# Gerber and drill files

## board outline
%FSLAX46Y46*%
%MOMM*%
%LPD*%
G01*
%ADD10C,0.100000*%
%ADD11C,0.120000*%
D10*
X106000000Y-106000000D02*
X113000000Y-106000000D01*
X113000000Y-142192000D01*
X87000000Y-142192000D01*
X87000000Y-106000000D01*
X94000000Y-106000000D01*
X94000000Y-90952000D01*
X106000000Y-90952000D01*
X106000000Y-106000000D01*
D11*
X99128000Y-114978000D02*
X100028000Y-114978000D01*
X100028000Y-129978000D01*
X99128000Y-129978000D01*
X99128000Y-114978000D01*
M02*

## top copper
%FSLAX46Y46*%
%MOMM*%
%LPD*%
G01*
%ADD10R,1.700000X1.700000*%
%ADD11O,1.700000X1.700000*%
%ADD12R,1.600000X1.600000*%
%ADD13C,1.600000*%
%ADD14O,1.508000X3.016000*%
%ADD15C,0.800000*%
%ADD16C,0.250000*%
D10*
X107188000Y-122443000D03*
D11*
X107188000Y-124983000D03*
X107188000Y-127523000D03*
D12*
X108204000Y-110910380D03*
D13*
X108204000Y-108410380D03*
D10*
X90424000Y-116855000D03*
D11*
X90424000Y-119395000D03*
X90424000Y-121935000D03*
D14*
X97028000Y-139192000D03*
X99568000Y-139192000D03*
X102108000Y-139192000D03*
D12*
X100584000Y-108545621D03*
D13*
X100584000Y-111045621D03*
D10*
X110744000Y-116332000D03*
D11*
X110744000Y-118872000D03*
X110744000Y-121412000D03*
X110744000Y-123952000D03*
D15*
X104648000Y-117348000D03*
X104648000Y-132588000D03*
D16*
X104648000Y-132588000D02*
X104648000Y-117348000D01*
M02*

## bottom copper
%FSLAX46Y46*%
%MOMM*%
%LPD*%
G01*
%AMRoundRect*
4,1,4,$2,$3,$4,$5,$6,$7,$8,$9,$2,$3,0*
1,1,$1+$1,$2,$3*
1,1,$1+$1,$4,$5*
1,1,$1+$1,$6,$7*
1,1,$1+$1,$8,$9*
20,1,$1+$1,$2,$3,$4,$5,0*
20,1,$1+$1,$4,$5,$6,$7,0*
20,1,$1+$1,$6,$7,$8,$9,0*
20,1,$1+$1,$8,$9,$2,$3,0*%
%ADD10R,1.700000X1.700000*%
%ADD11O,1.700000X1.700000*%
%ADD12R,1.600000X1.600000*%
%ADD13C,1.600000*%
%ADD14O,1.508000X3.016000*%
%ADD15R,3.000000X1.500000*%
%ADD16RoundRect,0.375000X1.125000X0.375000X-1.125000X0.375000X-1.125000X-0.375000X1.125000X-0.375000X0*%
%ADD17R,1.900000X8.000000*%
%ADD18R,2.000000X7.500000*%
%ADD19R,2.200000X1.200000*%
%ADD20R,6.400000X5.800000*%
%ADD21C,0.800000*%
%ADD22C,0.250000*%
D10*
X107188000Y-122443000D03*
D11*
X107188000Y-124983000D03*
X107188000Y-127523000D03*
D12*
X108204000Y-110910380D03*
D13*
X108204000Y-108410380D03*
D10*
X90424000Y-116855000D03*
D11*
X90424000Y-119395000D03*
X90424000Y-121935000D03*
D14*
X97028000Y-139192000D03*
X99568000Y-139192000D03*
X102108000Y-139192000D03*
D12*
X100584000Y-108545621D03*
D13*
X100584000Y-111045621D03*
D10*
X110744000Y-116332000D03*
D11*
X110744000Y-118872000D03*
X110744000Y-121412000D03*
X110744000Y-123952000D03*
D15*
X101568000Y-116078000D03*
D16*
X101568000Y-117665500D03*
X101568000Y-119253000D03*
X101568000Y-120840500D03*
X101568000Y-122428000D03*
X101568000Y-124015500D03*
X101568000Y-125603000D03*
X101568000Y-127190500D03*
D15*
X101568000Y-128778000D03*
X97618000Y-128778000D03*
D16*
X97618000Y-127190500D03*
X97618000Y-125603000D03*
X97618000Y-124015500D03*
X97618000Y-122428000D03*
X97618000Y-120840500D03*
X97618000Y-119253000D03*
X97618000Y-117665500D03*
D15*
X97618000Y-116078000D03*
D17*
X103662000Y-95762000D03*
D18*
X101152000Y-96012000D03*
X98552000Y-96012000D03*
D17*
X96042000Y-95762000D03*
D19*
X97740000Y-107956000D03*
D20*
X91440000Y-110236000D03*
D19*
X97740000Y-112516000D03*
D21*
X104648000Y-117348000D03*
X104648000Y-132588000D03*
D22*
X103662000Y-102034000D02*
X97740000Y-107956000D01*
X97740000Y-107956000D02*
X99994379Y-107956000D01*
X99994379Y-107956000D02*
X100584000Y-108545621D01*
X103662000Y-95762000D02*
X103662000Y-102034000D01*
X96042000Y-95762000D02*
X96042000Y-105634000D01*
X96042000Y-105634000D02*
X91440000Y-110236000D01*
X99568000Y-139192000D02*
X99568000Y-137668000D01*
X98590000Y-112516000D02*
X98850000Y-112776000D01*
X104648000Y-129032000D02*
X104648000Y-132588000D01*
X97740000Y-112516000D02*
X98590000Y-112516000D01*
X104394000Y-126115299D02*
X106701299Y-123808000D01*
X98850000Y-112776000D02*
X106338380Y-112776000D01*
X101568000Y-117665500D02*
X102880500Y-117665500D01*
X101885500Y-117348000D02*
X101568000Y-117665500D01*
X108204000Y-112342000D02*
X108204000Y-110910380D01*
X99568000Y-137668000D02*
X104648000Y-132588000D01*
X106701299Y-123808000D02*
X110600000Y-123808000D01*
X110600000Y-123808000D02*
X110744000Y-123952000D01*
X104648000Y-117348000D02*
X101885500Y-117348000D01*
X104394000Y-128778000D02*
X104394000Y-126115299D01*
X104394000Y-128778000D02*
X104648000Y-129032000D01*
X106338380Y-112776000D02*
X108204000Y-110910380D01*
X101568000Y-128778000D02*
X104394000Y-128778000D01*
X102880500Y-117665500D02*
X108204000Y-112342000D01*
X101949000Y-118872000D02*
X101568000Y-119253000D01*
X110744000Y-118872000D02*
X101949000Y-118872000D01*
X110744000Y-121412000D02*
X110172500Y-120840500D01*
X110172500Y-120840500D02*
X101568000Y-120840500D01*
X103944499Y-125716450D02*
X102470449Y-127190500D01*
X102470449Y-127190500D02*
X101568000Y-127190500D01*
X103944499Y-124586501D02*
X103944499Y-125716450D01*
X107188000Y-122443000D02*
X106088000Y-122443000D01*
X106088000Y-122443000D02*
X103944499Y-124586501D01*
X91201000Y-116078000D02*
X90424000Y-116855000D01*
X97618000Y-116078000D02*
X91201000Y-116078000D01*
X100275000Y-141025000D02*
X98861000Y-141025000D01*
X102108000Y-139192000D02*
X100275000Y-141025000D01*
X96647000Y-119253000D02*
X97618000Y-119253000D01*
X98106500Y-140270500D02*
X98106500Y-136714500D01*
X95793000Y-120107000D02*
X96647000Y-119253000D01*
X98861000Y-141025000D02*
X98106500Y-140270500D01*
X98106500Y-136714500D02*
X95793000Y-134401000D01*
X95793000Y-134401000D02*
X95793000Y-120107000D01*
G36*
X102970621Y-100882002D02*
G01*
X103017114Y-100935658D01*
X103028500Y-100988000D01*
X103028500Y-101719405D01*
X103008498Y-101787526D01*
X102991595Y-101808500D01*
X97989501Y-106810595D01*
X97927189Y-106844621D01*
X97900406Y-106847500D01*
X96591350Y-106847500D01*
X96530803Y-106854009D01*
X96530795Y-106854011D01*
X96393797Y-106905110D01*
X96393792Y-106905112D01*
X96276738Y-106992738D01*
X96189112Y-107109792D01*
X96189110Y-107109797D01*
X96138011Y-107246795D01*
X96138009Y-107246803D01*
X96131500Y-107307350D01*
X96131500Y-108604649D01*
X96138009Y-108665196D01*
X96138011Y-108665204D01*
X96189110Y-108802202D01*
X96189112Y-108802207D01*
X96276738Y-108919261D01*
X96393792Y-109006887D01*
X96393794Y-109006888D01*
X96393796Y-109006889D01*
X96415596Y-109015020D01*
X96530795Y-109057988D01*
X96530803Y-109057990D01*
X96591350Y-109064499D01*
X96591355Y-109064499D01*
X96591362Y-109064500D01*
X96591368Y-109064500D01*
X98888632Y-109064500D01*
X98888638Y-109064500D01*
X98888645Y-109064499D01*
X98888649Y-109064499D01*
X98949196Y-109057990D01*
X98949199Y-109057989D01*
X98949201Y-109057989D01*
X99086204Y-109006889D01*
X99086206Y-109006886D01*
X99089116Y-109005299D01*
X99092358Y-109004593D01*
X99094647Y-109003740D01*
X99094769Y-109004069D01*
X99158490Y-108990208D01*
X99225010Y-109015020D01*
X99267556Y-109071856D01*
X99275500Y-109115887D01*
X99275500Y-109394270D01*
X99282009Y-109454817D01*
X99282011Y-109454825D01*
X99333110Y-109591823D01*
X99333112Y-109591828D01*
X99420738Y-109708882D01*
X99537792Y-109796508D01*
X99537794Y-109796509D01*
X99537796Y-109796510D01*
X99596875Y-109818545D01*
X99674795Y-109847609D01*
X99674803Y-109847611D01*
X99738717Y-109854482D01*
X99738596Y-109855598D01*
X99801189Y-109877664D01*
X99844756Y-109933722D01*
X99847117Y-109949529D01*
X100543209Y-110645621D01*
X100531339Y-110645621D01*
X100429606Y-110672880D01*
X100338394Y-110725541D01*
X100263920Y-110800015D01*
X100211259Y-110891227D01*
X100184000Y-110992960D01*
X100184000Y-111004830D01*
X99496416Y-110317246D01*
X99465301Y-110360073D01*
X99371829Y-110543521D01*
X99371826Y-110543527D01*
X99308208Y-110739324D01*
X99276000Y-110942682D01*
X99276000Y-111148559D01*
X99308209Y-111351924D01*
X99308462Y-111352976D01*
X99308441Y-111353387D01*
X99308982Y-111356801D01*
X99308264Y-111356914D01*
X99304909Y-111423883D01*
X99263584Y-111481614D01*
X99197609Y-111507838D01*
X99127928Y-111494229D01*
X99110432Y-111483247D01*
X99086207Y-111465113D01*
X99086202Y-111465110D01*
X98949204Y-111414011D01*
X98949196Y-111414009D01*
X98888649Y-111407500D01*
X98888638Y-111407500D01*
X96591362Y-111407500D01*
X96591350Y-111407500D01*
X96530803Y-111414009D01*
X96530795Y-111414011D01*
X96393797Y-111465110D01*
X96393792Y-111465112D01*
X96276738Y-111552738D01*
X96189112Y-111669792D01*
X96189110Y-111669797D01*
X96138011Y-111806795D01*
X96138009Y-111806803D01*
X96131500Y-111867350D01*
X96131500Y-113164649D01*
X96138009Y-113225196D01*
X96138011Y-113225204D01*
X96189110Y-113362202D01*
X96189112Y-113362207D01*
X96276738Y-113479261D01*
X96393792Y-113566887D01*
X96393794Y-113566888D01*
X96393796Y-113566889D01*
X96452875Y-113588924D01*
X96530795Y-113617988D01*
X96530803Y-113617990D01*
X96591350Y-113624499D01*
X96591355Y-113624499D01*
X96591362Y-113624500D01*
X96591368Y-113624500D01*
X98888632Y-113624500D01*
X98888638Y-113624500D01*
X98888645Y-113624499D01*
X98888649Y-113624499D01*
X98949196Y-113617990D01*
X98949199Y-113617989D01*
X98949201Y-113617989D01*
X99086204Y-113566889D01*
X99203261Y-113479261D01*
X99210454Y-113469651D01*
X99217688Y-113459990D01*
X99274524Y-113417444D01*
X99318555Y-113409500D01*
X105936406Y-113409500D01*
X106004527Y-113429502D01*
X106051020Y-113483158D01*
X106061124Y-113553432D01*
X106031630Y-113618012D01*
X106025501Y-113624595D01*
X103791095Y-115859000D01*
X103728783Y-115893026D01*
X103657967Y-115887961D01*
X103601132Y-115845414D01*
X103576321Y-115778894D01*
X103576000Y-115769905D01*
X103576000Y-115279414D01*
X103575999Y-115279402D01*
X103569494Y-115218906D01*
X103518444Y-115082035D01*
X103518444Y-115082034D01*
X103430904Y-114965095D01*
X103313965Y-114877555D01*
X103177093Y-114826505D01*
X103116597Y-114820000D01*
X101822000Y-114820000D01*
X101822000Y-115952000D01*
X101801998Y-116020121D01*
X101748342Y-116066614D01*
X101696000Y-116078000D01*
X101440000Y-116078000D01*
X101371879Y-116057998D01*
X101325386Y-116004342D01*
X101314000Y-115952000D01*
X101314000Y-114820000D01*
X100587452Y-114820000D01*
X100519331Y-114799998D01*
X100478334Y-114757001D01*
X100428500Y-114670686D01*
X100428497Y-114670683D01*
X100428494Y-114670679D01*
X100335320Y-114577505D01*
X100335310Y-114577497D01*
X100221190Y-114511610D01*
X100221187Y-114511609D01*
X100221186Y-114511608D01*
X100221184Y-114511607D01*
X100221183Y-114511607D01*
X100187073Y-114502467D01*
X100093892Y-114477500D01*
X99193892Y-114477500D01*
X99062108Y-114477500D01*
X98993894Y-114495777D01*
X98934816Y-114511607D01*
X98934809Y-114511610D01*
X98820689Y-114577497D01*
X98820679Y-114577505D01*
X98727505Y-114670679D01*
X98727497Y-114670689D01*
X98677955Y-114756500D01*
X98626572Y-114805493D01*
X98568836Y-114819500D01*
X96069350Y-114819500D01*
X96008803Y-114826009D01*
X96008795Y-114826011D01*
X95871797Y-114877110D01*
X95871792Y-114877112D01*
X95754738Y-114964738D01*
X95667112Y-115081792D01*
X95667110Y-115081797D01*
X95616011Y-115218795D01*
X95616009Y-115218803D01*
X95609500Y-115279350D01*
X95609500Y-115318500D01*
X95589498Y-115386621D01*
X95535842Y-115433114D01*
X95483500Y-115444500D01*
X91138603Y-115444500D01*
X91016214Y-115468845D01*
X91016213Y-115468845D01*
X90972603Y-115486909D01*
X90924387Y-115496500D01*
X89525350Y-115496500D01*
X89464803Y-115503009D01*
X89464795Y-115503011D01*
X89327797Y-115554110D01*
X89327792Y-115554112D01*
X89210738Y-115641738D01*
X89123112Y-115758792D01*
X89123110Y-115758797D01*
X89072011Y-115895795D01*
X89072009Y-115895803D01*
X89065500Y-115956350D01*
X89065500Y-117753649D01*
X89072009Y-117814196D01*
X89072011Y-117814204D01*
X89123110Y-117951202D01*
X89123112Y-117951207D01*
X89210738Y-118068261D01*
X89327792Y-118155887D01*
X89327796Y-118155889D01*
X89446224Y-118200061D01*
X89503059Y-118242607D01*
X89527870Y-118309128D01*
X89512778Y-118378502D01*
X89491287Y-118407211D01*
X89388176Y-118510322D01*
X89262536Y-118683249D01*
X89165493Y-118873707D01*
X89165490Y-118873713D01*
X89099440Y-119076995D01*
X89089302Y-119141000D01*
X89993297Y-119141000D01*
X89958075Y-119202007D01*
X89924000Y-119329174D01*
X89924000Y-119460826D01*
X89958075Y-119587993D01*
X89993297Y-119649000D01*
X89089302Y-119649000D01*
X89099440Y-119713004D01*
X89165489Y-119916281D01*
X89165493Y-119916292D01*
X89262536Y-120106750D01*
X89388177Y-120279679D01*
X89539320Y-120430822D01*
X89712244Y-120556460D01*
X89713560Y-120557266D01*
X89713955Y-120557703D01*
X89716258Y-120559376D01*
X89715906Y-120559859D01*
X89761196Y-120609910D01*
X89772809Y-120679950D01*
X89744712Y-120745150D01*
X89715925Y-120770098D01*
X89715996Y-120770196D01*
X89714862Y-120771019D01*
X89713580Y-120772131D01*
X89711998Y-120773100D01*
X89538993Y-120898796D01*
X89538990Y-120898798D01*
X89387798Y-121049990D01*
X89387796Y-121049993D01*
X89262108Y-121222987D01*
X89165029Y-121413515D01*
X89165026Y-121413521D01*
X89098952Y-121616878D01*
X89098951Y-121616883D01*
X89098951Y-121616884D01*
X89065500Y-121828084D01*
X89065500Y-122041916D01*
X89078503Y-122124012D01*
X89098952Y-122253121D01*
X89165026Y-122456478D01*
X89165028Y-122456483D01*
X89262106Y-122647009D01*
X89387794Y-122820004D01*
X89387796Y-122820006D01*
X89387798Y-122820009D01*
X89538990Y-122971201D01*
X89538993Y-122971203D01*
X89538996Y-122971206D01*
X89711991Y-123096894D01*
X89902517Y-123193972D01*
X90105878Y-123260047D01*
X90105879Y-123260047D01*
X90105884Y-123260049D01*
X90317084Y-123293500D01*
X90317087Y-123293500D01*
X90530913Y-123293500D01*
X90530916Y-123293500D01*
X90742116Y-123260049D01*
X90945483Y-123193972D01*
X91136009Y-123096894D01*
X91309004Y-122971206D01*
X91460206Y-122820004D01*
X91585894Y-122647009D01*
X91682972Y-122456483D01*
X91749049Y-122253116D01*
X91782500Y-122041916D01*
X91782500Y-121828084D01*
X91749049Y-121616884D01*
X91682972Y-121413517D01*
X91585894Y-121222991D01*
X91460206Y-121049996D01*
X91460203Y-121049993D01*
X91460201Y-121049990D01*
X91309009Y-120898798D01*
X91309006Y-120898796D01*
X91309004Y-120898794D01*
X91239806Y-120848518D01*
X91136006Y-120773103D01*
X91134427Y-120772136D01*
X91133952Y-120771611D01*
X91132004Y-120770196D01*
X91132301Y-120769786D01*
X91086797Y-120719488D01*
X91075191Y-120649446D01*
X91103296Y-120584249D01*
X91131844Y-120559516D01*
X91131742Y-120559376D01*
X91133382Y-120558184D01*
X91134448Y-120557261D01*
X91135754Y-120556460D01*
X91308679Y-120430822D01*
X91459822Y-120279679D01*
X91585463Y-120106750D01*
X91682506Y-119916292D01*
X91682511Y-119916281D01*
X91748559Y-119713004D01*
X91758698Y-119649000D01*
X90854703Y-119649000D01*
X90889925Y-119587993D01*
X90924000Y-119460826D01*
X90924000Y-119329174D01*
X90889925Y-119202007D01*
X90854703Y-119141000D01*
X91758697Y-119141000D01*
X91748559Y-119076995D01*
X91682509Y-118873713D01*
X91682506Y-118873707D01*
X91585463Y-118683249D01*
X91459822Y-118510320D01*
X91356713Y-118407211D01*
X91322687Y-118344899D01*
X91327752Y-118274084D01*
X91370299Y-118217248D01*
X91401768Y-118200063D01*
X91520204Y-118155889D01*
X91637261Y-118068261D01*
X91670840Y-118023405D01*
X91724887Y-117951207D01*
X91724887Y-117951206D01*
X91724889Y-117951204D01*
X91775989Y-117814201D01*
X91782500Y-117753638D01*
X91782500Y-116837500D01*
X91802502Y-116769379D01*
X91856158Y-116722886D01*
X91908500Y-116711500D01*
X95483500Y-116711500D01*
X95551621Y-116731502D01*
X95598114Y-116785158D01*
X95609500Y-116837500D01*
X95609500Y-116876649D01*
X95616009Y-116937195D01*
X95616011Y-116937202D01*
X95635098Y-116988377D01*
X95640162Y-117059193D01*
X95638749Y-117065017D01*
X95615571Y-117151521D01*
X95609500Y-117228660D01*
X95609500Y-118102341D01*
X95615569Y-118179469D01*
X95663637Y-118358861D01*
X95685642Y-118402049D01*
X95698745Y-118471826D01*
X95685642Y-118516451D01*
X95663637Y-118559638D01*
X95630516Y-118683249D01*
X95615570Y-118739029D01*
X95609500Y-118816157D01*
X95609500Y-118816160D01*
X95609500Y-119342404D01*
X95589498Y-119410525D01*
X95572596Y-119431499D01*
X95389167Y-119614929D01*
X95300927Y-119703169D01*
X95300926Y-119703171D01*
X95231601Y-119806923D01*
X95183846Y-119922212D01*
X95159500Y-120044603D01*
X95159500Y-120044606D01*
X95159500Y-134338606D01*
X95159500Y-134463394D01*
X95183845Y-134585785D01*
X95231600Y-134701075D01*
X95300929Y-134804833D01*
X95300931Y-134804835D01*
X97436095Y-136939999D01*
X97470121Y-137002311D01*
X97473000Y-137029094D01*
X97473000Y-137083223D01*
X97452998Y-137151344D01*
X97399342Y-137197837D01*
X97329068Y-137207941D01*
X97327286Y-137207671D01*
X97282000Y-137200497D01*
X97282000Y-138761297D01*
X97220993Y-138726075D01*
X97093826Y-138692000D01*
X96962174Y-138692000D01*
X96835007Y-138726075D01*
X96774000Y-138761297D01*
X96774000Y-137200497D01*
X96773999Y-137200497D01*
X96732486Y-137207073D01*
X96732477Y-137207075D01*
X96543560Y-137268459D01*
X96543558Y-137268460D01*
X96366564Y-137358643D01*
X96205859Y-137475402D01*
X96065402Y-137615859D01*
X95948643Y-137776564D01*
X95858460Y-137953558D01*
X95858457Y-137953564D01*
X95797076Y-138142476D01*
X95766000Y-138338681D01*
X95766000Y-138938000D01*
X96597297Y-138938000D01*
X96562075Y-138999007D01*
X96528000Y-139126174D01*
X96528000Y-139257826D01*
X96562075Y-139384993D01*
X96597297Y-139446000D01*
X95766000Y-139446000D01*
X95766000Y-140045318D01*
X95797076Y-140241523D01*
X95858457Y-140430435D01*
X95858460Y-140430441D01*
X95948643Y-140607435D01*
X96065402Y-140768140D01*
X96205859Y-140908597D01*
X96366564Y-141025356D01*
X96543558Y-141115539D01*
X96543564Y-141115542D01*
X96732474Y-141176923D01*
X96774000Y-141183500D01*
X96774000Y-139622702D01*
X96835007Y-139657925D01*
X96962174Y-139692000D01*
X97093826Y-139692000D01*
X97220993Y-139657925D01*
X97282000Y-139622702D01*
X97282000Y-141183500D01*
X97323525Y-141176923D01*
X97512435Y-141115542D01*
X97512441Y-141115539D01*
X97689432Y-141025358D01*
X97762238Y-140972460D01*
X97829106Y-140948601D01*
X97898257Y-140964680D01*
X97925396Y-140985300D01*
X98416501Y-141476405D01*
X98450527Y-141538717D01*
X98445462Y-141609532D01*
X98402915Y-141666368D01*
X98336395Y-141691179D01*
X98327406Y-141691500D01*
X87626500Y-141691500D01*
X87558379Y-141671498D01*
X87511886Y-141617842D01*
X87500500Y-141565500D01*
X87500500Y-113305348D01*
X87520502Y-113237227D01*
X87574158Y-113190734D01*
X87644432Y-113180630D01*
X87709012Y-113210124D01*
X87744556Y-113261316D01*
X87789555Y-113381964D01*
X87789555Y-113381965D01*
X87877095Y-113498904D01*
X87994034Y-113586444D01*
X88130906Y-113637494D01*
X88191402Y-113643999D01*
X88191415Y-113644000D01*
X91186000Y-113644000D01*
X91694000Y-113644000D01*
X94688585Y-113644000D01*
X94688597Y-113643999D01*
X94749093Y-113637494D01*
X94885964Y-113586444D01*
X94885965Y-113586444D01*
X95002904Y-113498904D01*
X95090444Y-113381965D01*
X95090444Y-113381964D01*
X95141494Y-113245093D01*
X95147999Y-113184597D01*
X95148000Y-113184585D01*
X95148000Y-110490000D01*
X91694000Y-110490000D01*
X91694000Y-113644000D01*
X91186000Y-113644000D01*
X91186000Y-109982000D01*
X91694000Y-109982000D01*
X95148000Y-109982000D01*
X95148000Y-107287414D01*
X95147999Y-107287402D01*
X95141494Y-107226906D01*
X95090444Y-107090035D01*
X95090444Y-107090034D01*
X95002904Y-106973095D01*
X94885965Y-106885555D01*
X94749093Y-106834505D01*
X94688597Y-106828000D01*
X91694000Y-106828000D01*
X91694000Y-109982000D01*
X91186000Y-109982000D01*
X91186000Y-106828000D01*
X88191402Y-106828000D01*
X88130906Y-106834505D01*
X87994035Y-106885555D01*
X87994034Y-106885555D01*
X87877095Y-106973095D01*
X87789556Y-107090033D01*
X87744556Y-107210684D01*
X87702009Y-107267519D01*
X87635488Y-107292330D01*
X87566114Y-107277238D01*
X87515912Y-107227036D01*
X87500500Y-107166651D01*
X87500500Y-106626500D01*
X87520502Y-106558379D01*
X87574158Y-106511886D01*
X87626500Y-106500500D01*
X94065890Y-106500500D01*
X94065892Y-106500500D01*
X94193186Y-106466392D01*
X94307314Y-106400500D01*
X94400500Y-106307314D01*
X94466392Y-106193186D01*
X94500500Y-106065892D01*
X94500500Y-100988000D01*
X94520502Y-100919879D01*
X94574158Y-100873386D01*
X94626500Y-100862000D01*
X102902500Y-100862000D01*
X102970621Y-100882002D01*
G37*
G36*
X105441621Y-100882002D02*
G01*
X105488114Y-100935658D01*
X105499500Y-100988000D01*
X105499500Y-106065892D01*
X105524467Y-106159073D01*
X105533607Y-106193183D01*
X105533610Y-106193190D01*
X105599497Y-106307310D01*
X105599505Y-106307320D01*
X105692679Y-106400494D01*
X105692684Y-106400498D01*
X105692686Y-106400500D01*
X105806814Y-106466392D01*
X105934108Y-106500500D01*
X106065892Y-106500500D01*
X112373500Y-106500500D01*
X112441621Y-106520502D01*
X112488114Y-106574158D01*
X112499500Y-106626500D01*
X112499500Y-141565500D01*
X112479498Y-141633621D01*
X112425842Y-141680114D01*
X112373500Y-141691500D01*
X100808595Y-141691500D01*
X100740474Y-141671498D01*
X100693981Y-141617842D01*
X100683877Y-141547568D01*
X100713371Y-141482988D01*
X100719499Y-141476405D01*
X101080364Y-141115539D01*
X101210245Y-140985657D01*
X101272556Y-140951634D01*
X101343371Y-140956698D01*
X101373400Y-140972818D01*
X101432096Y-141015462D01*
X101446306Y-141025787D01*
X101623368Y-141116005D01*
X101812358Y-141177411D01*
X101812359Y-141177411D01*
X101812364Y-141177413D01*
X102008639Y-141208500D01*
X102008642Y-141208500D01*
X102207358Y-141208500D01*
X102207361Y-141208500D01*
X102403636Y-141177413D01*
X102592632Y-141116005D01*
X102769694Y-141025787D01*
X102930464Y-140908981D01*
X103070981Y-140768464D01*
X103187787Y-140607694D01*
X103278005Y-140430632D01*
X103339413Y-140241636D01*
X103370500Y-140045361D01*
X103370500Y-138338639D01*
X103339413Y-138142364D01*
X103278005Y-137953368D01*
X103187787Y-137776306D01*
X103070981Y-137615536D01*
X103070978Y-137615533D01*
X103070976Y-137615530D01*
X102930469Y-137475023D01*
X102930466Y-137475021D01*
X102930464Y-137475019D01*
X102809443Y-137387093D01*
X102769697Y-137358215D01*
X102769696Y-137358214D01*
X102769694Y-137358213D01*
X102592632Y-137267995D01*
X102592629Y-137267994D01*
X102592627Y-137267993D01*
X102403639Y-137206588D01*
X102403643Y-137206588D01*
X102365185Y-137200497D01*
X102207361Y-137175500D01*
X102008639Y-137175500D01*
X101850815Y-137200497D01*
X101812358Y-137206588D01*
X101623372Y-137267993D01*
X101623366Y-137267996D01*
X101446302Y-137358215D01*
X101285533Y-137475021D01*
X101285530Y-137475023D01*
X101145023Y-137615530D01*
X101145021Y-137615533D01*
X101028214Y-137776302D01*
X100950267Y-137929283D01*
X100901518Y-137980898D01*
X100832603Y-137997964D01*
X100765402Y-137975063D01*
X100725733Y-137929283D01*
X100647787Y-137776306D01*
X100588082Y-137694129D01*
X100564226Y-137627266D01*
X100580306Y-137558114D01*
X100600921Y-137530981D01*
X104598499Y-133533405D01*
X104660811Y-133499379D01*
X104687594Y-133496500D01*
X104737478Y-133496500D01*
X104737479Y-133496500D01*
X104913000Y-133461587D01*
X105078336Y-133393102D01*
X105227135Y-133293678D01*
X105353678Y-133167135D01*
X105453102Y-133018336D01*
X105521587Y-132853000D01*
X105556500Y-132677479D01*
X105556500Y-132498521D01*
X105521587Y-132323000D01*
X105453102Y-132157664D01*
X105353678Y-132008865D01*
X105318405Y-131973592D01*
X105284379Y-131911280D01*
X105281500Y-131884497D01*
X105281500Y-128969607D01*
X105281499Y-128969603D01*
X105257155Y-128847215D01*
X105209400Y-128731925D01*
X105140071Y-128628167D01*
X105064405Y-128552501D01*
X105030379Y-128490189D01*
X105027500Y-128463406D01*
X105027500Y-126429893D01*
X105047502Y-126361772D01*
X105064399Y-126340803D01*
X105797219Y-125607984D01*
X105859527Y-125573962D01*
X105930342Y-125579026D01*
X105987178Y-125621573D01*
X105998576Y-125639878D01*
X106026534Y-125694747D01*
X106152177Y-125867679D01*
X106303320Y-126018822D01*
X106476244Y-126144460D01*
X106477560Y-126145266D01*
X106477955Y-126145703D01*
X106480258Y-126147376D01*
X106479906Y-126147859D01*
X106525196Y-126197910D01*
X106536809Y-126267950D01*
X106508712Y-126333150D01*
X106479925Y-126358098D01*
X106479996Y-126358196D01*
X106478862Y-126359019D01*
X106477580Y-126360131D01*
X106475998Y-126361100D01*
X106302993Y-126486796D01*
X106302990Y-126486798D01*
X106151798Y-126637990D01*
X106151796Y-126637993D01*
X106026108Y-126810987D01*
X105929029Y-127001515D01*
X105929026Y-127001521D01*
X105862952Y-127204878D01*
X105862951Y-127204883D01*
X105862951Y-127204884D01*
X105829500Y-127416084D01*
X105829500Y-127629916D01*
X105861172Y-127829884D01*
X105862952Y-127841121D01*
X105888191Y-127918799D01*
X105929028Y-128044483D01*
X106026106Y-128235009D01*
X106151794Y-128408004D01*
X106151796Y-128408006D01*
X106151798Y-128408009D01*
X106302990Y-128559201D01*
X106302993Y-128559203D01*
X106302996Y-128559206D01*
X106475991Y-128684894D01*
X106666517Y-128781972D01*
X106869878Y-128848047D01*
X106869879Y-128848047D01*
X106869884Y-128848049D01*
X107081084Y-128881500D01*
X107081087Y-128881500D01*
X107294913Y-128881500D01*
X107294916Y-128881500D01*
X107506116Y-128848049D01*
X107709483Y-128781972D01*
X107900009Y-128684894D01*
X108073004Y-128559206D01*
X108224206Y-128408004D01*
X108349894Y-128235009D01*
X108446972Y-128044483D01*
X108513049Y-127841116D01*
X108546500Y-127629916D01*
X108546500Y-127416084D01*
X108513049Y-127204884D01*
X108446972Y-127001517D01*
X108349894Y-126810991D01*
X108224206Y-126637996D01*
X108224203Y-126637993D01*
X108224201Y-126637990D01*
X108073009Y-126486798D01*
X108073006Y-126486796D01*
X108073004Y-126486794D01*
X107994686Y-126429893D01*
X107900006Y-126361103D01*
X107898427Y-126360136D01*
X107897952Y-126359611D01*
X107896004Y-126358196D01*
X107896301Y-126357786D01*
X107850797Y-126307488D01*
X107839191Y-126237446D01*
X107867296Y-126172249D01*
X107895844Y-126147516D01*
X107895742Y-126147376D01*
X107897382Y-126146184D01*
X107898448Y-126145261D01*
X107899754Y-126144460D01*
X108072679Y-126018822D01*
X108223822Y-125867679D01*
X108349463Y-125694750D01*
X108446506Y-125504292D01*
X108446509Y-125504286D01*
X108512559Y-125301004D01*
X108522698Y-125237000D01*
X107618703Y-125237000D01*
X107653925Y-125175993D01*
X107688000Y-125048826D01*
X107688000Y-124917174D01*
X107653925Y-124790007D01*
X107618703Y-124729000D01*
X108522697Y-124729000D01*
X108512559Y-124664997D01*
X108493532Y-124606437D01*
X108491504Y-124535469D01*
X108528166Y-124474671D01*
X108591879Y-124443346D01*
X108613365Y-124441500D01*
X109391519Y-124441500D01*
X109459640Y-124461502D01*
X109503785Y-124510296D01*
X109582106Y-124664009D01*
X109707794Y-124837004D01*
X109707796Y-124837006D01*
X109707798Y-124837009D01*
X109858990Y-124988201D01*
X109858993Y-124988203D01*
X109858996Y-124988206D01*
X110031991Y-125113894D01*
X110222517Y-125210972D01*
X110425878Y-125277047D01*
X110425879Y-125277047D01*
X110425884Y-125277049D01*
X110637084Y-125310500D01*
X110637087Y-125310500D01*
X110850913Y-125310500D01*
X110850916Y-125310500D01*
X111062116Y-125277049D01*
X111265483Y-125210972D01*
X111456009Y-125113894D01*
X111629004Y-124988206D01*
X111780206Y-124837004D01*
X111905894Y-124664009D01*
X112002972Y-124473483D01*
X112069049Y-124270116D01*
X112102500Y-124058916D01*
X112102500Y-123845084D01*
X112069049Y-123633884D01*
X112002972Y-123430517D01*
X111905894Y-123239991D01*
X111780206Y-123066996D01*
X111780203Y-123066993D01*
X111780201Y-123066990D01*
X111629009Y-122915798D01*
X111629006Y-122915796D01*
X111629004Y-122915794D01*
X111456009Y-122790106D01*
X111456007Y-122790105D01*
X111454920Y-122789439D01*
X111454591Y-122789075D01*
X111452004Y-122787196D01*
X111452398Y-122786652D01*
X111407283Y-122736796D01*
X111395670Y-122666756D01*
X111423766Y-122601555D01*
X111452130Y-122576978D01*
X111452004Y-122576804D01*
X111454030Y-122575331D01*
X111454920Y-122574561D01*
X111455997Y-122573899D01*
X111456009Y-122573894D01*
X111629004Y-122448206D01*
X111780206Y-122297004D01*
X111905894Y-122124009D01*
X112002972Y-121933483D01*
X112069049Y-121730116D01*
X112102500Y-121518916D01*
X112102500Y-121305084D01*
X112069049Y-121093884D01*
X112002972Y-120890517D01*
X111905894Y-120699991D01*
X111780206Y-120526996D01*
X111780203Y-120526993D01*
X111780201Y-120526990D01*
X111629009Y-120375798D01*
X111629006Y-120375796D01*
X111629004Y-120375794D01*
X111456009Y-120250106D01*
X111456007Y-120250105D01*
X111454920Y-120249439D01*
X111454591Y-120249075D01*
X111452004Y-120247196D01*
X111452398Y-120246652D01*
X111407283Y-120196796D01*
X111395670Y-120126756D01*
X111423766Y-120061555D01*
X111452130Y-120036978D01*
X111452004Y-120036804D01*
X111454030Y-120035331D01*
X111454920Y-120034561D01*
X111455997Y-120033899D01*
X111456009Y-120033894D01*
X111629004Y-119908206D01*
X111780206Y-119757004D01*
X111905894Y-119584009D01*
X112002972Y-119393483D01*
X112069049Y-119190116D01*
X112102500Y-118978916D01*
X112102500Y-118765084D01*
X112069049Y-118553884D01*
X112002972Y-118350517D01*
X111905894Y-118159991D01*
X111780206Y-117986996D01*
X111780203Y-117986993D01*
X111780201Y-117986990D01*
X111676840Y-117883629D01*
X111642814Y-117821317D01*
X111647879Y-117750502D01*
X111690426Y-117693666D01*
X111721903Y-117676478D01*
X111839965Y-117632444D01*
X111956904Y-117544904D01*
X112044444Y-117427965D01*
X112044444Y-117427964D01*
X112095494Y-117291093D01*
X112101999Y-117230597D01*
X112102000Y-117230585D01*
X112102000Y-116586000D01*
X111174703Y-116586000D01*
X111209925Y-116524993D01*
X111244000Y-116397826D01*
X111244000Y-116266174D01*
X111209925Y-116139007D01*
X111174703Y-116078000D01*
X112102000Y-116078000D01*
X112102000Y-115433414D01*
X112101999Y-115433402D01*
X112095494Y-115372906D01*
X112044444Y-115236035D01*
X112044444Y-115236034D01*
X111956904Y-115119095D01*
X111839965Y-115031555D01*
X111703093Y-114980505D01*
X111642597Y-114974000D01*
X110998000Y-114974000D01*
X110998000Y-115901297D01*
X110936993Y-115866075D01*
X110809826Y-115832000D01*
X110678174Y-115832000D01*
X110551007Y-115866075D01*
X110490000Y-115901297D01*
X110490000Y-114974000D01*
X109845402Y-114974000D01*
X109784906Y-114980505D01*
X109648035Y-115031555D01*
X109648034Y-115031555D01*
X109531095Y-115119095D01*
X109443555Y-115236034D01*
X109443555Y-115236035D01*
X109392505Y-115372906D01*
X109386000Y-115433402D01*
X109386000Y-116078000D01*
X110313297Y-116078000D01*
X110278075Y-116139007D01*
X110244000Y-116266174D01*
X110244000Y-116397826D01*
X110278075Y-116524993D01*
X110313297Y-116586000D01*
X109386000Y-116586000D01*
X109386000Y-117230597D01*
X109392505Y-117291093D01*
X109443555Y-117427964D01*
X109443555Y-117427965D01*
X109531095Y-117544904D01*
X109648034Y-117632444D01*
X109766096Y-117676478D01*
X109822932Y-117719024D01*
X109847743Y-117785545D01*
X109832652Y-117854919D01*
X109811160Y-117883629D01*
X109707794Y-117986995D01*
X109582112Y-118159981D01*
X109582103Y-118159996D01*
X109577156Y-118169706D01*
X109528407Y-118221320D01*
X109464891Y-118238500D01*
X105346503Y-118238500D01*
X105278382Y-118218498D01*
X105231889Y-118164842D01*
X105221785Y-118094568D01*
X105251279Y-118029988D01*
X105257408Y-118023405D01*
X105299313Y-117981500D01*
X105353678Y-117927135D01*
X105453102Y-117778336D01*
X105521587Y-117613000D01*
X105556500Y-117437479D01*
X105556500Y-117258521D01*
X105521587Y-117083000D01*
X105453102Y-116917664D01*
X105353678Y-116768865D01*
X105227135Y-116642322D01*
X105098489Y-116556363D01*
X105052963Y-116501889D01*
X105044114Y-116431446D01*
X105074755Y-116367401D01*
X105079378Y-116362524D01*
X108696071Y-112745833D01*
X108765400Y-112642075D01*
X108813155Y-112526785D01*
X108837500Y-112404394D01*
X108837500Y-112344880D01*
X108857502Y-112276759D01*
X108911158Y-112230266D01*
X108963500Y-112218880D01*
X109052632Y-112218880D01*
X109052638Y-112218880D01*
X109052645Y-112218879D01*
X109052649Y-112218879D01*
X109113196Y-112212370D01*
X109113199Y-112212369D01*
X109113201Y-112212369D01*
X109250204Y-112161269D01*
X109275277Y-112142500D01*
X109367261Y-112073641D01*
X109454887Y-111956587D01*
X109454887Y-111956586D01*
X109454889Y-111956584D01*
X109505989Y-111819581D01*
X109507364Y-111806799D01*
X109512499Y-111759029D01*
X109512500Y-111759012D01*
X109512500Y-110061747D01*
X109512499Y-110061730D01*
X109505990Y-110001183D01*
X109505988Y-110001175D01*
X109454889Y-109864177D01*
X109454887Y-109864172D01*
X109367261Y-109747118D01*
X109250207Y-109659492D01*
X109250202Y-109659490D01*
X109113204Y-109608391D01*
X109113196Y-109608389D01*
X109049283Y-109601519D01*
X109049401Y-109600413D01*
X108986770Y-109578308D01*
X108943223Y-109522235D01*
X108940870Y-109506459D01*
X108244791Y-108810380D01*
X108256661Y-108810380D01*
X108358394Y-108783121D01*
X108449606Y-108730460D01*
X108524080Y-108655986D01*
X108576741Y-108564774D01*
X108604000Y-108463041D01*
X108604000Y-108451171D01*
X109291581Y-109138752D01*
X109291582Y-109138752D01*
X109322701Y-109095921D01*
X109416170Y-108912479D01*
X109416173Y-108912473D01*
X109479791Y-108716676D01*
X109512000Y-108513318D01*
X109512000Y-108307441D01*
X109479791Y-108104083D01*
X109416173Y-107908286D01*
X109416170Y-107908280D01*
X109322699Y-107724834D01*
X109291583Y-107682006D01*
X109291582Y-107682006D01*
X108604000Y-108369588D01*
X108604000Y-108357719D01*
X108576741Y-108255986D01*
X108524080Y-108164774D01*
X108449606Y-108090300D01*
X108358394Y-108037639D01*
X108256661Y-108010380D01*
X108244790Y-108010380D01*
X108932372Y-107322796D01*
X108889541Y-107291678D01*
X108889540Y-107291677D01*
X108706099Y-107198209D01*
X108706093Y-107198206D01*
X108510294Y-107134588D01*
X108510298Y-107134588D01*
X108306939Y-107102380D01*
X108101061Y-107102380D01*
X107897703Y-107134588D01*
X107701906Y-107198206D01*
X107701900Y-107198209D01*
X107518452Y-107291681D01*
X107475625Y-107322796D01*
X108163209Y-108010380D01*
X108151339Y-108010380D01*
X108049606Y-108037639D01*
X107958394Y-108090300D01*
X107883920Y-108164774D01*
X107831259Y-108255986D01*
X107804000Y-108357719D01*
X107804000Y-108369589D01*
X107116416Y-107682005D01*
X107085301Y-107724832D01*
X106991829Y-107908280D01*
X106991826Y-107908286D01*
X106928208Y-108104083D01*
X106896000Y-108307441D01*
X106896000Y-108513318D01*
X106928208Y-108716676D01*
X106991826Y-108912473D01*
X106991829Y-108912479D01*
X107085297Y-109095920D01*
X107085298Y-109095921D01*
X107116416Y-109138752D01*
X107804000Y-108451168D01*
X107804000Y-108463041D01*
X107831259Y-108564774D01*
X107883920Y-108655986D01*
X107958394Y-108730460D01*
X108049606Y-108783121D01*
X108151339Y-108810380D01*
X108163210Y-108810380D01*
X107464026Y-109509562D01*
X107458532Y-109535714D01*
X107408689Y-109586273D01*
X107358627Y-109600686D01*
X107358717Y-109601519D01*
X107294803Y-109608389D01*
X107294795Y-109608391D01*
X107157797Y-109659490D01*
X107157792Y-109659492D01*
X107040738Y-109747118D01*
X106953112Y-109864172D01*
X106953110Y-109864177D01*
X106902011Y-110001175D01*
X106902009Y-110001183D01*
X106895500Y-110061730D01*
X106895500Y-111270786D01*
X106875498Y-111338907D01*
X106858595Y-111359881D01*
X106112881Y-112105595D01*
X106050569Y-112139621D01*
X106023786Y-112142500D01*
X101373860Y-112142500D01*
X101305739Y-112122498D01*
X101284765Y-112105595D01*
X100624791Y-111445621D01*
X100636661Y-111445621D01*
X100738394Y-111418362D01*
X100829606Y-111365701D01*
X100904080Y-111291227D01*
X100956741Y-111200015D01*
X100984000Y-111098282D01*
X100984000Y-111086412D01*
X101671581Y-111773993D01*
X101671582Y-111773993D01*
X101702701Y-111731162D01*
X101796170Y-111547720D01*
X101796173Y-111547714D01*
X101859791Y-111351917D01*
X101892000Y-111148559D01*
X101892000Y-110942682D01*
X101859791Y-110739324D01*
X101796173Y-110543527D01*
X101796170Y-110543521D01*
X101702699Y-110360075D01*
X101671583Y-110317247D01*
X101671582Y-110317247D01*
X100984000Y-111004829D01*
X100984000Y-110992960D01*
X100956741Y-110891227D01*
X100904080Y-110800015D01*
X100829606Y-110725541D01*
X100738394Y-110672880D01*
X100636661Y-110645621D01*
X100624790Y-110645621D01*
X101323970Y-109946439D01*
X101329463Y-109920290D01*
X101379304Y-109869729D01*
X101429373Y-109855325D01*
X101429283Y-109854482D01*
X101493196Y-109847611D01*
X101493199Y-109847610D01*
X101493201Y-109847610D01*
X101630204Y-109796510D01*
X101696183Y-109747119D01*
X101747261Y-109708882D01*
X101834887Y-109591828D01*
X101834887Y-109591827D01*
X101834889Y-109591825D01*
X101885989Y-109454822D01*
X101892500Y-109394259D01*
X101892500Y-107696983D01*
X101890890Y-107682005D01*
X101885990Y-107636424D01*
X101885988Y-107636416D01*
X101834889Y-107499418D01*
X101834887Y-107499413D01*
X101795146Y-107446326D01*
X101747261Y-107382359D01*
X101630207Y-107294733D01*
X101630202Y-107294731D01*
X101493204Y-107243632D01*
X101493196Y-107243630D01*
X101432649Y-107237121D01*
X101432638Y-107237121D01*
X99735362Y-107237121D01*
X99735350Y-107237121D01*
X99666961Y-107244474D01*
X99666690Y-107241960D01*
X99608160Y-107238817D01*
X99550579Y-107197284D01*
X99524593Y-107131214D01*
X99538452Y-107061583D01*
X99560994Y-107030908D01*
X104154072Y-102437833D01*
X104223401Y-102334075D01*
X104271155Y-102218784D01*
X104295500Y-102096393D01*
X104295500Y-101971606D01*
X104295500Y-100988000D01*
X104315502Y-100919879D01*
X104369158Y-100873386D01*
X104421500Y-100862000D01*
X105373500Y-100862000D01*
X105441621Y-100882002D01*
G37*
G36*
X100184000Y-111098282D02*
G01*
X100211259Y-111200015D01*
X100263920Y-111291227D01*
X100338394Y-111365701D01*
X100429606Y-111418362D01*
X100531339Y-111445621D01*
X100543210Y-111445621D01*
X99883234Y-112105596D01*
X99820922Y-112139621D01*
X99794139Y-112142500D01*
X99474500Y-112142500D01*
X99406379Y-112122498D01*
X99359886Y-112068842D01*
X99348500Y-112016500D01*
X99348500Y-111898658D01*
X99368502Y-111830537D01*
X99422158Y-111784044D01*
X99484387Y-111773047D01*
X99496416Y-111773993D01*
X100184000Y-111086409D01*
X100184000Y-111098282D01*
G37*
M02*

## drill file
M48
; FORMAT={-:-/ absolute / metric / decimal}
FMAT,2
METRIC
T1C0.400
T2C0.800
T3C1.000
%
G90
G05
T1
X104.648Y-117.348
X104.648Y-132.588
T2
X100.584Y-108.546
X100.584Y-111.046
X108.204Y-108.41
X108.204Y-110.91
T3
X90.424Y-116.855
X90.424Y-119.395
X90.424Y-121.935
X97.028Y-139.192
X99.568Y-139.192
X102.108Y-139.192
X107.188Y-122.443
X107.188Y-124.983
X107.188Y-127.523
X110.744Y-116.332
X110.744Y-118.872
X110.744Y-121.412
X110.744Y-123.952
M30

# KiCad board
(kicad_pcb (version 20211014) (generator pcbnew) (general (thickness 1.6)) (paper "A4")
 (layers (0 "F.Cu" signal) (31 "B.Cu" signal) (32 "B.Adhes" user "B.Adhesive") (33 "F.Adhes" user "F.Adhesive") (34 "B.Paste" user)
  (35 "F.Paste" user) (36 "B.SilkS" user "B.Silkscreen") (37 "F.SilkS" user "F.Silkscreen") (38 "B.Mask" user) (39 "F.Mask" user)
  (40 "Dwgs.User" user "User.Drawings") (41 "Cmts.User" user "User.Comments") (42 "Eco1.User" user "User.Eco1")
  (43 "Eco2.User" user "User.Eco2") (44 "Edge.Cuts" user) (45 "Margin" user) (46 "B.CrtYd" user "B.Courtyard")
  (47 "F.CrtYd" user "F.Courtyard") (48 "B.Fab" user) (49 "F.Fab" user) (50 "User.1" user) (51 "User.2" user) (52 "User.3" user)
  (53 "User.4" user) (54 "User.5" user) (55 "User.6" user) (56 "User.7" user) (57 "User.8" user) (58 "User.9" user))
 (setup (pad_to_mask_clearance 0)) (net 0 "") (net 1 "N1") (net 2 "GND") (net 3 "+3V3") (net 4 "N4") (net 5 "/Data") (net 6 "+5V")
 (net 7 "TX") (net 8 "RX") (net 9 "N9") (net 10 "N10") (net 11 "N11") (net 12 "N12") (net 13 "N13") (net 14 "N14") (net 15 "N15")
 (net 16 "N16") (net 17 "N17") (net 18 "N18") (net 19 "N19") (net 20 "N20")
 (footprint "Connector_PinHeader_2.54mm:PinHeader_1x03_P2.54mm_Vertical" (layer "F.Cu") (at 107.188 122.443)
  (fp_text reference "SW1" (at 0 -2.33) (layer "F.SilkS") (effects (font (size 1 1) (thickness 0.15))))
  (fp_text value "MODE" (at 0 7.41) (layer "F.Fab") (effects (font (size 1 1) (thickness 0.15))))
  (pad "1" thru_hole rect (at 0 0) (size 1.7 1.7) (drill 1) (layers *.Cu *.Mask) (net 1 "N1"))
  (pad "2" thru_hole oval (at 0 2.54) (size 1.7 1.7) (drill 1) (layers *.Cu *.Mask) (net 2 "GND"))
  (pad "3" thru_hole oval (at 0 5.08) (size 1.7 1.7) (drill 1) (layers *.Cu *.Mask)))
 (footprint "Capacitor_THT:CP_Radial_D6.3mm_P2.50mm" (layer "F.Cu") (at 108.204 110.91038 90)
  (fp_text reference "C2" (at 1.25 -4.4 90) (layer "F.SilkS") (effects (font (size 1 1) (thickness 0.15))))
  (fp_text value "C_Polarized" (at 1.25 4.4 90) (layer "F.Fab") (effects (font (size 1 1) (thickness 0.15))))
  (pad "1" thru_hole rect (at 0 0 90) (size 1.6 1.6) (drill 0.8) (layers *.Cu *.Mask) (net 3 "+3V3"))
  (pad "2" thru_hole circle (at 2.5 0 90) (size 1.6 1.6) (drill 0.8) (layers *.Cu *.Mask) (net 2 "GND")))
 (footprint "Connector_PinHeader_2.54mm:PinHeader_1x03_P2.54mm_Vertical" (layer "F.Cu") (at 90.424 116.855)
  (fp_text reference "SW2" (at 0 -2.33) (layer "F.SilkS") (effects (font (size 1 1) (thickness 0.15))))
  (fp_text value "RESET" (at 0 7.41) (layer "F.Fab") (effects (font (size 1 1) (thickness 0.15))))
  (pad "1" thru_hole rect (at 0 0) (size 1.7 1.7) (drill 1) (layers *.Cu *.Mask) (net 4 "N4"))
  (pad "2" thru_hole oval (at 0 2.54) (size 1.7 1.7) (drill 1) (layers *.Cu *.Mask) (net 2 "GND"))
  (pad "3" thru_hole oval (at 0 5.08) (size 1.7 1.7) (drill 1) (layers *.Cu *.Mask)))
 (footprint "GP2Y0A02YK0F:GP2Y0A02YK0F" (layer "F.Cu") (at 99.568 139.192)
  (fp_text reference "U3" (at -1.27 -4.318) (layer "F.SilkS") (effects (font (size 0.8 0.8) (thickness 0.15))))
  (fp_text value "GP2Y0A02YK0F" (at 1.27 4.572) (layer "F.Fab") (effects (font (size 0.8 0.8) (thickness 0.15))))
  (pad "1" thru_hole oval (at -2.54 0) (size 1.508 3.016) (drill 1) (layers *.Cu *.Mask) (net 2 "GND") (solder_mask_margin 0.102))
  (pad "2" thru_hole oval (at 0 0) (size 1.508 3.016) (drill 1) (layers *.Cu *.Mask) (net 3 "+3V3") (solder_mask_margin 0.102))
  (pad "3" thru_hole oval (at 2.54 0) (size 1.508 3.016) (drill 1) (layers *.Cu *.Mask) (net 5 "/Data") (solder_mask_margin 0.102)))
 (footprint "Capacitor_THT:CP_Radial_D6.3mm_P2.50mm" (layer "F.Cu") (at 100.584 108.545621 -90)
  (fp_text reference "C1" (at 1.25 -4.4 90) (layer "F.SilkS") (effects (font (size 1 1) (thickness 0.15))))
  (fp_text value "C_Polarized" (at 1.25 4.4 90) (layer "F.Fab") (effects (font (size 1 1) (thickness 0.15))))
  (pad "1" thru_hole rect (at 0 0 270) (size 1.6 1.6) (drill 0.8) (layers *.Cu *.Mask) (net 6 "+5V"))
  (pad "2" thru_hole circle (at 2.5 0 270) (size 1.6 1.6) (drill 0.8) (layers *.Cu *.Mask) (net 2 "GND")))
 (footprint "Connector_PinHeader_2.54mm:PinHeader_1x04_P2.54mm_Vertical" (layer "F.Cu") (at 110.744 116.332)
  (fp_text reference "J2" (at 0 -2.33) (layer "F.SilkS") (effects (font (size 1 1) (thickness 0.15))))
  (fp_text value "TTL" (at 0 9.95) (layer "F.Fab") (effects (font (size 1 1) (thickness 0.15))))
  (pad "1" thru_hole rect (at 0 0) (size 1.7 1.7) (drill 1) (layers *.Cu *.Mask) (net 2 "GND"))
  (pad "2" thru_hole oval (at 0 2.54) (size 1.7 1.7) (drill 1) (layers *.Cu *.Mask) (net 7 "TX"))
  (pad "3" thru_hole oval (at 0 5.08) (size 1.7 1.7) (drill 1) (layers *.Cu *.Mask) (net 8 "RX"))
  (pad "4" thru_hole oval (at 0 7.62) (size 1.7 1.7) (drill 1) (layers *.Cu *.Mask) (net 3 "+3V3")))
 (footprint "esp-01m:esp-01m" (layer "B.Cu") (at 99.568 122.428 180)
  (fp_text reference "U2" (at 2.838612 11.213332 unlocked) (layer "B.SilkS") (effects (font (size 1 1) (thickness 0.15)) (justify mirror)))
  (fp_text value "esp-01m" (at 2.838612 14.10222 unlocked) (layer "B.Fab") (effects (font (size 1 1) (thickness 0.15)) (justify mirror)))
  (fp_rect (start -0.46 7.45) (end 0.44 -7.55) (layer "Edge.Cuts") (width 0.12) (fill none))
  (pad "1" smd rect (at -2 6.35 180) (size 3 1.5) (layers "B.Cu" "B.Paste" "B.Mask") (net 2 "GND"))
  (pad "2" smd roundrect (at -2 4.7625 180) (size 3 1.5) (layers "B.Cu" "B.Paste" "B.Mask") (roundrect_rratio 0.25) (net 3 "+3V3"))
  (pad "3" smd roundrect (at -2 3.175 180) (size 3 1.5) (layers "B.Cu" "B.Paste" "B.Mask") (roundrect_rratio 0.25) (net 7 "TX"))
  (pad "4" smd roundrect (at -2 1.5875 180) (size 3 1.5) (layers "B.Cu" "B.Paste" "B.Mask") (roundrect_rratio 0.25) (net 8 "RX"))
  (pad "5" smd roundrect (at -2 0 180) (size 3 1.5) (layers "B.Cu" "B.Paste" "B.Mask") (roundrect_rratio 0.25) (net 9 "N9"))
  (pad "6" smd roundrect (at -2 -1.5875 180) (size 3 1.5) (layers "B.Cu" "B.Paste" "B.Mask") (roundrect_rratio 0.25) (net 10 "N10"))
  (pad "7" smd roundrect (at -2 -3.175 180) (size 3 1.5) (layers "B.Cu" "B.Paste" "B.Mask") (roundrect_rratio 0.25) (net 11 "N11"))
  (pad "8" smd roundrect (at -2 -4.7625 180) (size 3 1.5) (layers "B.Cu" "B.Paste" "B.Mask") (roundrect_rratio 0.25) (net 1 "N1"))
  (pad "9" smd rect (at -2 -6.35 180) (size 3 1.5) (layers "B.Cu" "B.Paste" "B.Mask") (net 3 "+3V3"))
  (pad "10" smd rect (at 1.95 -6.35 180) (size 3 1.5) (layers "B.Cu" "B.Paste" "B.Mask") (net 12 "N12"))
  (pad "11" smd roundrect (at 1.95 -4.7625 180) (size 3 1.5) (layers "B.Cu" "B.Paste" "B.Mask") (roundrect_rratio 0.25) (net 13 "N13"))
  (pad "12" smd roundrect (at 1.95 -3.175 180) (size 3 1.5) (layers "B.Cu" "B.Paste" "B.Mask") (roundrect_rratio 0.25) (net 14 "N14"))
  (pad "13" smd roundrect (at 1.95 -1.5875 180) (size 3 1.5) (layers "B.Cu" "B.Paste" "B.Mask") (roundrect_rratio 0.25) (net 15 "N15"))
  (pad "14" smd roundrect (at 1.95 0 180) (size 3 1.5) (layers "B.Cu" "B.Paste" "B.Mask") (roundrect_rratio 0.25) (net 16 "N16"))
  (pad "15" smd roundrect (at 1.95 1.5875 180) (size 3 1.5) (layers "B.Cu" "B.Paste" "B.Mask") (roundrect_rratio 0.25) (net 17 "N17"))
  (pad "16" smd roundrect (at 1.95 3.175 180) (size 3 1.5) (layers "B.Cu" "B.Paste" "B.Mask") (roundrect_rratio 0.25) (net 5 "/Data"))
  (pad "17" smd roundrect (at 1.95 4.7625 180) (size 3 1.5) (layers "B.Cu" "B.Paste" "B.Mask") (roundrect_rratio 0.25) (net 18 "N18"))
  (pad "18" smd rect (at 1.95 6.35 180) (size 3 1.5) (layers "B.Cu" "B.Paste" "B.Mask") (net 4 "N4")))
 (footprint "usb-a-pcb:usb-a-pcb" (layer "B.Cu") (at 99.852 90.862 180)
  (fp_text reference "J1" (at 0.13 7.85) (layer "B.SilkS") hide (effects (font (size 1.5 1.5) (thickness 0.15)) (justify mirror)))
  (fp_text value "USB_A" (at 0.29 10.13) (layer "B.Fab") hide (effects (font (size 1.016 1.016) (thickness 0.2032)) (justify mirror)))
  (pad "1" connect rect (at -3.81 -4.9) (size 1.9 8) (layers "B.Cu" "B.Mask") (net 6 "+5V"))
  (pad "2" connect rect (at -1.3 -5.15) (size 2 7.5) (layers "B.Cu" "B.Mask") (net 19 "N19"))
  (pad "3" connect rect (at 1.3 -5.15) (size 2 7.5) (layers "B.Cu" "B.Mask") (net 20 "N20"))
  (pad "4" connect rect (at 3.81 -4.9) (size 1.9 8) (layers "B.Cu" "B.Mask") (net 2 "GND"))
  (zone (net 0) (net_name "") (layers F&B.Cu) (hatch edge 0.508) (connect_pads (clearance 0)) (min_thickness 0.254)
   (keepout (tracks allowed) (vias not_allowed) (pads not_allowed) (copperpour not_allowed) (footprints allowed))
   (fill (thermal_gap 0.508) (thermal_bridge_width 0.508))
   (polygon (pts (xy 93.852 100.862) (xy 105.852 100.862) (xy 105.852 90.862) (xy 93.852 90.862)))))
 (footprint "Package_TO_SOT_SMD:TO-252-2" (layer "B.Cu") (at 93.54 110.236 180)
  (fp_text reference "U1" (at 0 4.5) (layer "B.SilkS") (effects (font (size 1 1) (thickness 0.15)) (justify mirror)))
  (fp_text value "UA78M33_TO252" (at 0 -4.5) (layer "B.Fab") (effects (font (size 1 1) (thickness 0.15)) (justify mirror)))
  (pad "" smd rect (at 3.775 1.525 180) (size 3.05 2.75) (layers "B.Paste"))
  (pad "" smd rect (at 0.425 -1.525 180) (size 3.05 2.75) (layers "B.Paste"))
  (pad "" smd rect (at 3.775 -1.525 180) (size 3.05 2.75) (layers "B.Paste"))
  (pad "" smd rect (at 0.425 1.525 180) (size 3.05 2.75) (layers "B.Paste"))
  (pad "1" smd rect (at -4.2 2.28 180) (size 2.2 1.2) (layers "B.Cu" "B.Paste" "B.Mask") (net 6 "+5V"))
  (pad "2" smd rect (at 2.1 0 180) (size 6.4 5.8) (layers "B.Cu" "B.Mask") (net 2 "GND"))
  (pad "3" smd rect (at -4.2 -2.28 180) (size 2.2 1.2) (layers "B.Cu" "B.Paste" "B.Mask") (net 3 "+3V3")))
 (gr_poly
  (pts (xy 106 106) (xy 113 106) (xy 113 142.192) (xy 87 142.192) (xy 87 106) (xy 94 106) (xy 94 90.952) (xy 106 90.952))
  (layer "Edge.Cuts") (width 0.1) (fill none))
 (segment (start 103.662 102.034) (end 97.74 107.956) (width 0.25) (layer "B.Cu") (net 6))
 (segment (start 97.74 107.956) (end 99.994379 107.956) (width 0.25) (layer "B.Cu") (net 6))
 (segment (start 99.994379 107.956) (end 100.584 108.545621) (width 0.25) (layer "B.Cu") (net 6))
 (segment (start 103.662 95.762) (end 103.662 102.034) (width 0.25) (layer "B.Cu") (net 6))
 (segment (start 96.042 95.762) (end 96.042 105.634) (width 0.25) (layer "B.Cu") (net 2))
 (segment (start 96.042 105.634) (end 91.44 110.236) (width 0.25) (layer "B.Cu") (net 2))
 (segment (start 104.648 132.588) (end 104.648 117.348) (width 0.25) (layer "F.Cu") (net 3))
 (via (at 104.648 117.348) (size 0.8) (drill 0.4) (layers "F.Cu" "B.Cu") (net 3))
 (via (at 104.648 132.588) (size 0.8) (drill 0.4) (layers "F.Cu" "B.Cu") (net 3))
 (segment (start 99.568 139.192) (end 99.568 137.668) (width 0.25) (layer "B.Cu") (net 3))
 (segment (start 98.59 112.516) (end 98.85 112.776) (width 0.25) (layer "B.Cu") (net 3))
 (segment (start 104.648 129.032) (end 104.648 132.588) (width 0.25) (layer "B.Cu") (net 3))
 (segment (start 97.74 112.516) (end 98.59 112.516) (width 0.25) (layer "B.Cu") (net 3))
 (segment (start 104.394 126.115299) (end 106.701299 123.808) (width 0.25) (layer "B.Cu") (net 3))
 (segment (start 98.85 112.776) (end 106.33838 112.776) (width 0.25) (layer "B.Cu") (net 3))
 (segment (start 101.568 117.6655) (end 102.8805 117.6655) (width 0.25) (layer "B.Cu") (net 3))
 (segment (start 101.8855 117.348) (end 101.568 117.6655) (width 0.25) (layer "B.Cu") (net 3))
 (segment (start 108.204 112.342) (end 108.204 110.91038) (width 0.25) (layer "B.Cu") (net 3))
 (segment (start 99.568 137.668) (end 104.648 132.588) (width 0.25) (layer "B.Cu") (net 3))
 (segment (start 106.701299 123.808) (end 110.6 123.808) (width 0.25) (layer "B.Cu") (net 3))
 (segment (start 110.6 123.808) (end 110.744 123.952) (width 0.25) (layer "B.Cu") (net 3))
 (segment (start 104.648 117.348) (end 101.8855 117.348) (width 0.25) (layer "B.Cu") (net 3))
 (segment (start 104.394 128.778) (end 104.394 126.115299) (width 0.25) (layer "B.Cu") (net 3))
 (segment (start 104.394 128.778) (end 104.648 129.032) (width 0.25) (layer "B.Cu") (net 3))
 (segment (start 106.33838 112.776) (end 108.204 110.91038) (width 0.25) (layer "B.Cu") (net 3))
 (segment (start 101.568 128.778) (end 104.394 128.778) (width 0.25) (layer "B.Cu") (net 3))
 (segment (start 102.8805 117.6655) (end 108.204 112.342) (width 0.25) (layer "B.Cu") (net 3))
 (segment (start 101.949 118.872) (end 101.568 119.253) (width 0.25) (layer "B.Cu") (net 7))
 (segment (start 110.744 118.872) (end 101.949 118.872) (width 0.25) (layer "B.Cu") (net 7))
 (segment (start 110.744 121.412) (end 110.1725 120.8405) (width 0.25) (layer "B.Cu") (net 8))
 (segment (start 110.1725 120.8405) (end 101.568 120.8405) (width 0.25) (layer "B.Cu") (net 8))
 (segment (start 103.944499 125.71645) (end 102.470449 127.1905) (width 0.25) (layer "B.Cu") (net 1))
 (segment (start 102.470449 127.1905) (end 101.568 127.1905) (width 0.25) (layer "B.Cu") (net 1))
 (segment (start 103.944499 124.586501) (end 103.944499 125.71645) (width 0.25) (layer "B.Cu") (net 1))
 (segment (start 107.188 122.443) (end 106.088 122.443) (width 0.25) (layer "B.Cu") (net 1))
 (segment (start 106.088 122.443) (end 103.944499 124.586501) (width 0.25) (layer "B.Cu") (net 1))
 (segment (start 91.201 116.078) (end 90.424 116.855) (width 0.25) (layer "B.Cu") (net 4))
 (segment (start 97.618 116.078) (end 91.201 116.078) (width 0.25) (layer "B.Cu") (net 4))
 (segment (start 100.275 141.025) (end 98.861 141.025) (width 0.25) (layer "B.Cu") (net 5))
 (segment (start 102.108 139.192) (end 100.275 141.025) (width 0.25) (layer "B.Cu") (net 5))
 (segment (start 96.647 119.253) (end 97.618 119.253) (width 0.25) (layer "B.Cu") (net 5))
 (segment (start 98.1065 140.2705) (end 98.1065 136.7145) (width 0.25) (layer "B.Cu") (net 5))
 (segment (start 95.793 120.107) (end 96.647 119.253) (width 0.25) (layer "B.Cu") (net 5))
 (segment (start 98.861 141.025) (end 98.1065 140.2705) (width 0.25) (layer "B.Cu") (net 5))
 (segment (start 98.1065 136.7145) (end 95.793 134.401) (width 0.25) (layer "B.Cu") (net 5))
 (segment (start 95.793 134.401) (end 95.793 120.107) (width 0.25) (layer "B.Cu") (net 5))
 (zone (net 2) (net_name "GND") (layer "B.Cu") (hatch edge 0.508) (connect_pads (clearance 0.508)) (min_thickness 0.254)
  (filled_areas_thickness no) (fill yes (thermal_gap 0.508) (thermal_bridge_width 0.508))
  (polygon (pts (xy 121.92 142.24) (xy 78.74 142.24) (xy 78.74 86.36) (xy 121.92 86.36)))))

